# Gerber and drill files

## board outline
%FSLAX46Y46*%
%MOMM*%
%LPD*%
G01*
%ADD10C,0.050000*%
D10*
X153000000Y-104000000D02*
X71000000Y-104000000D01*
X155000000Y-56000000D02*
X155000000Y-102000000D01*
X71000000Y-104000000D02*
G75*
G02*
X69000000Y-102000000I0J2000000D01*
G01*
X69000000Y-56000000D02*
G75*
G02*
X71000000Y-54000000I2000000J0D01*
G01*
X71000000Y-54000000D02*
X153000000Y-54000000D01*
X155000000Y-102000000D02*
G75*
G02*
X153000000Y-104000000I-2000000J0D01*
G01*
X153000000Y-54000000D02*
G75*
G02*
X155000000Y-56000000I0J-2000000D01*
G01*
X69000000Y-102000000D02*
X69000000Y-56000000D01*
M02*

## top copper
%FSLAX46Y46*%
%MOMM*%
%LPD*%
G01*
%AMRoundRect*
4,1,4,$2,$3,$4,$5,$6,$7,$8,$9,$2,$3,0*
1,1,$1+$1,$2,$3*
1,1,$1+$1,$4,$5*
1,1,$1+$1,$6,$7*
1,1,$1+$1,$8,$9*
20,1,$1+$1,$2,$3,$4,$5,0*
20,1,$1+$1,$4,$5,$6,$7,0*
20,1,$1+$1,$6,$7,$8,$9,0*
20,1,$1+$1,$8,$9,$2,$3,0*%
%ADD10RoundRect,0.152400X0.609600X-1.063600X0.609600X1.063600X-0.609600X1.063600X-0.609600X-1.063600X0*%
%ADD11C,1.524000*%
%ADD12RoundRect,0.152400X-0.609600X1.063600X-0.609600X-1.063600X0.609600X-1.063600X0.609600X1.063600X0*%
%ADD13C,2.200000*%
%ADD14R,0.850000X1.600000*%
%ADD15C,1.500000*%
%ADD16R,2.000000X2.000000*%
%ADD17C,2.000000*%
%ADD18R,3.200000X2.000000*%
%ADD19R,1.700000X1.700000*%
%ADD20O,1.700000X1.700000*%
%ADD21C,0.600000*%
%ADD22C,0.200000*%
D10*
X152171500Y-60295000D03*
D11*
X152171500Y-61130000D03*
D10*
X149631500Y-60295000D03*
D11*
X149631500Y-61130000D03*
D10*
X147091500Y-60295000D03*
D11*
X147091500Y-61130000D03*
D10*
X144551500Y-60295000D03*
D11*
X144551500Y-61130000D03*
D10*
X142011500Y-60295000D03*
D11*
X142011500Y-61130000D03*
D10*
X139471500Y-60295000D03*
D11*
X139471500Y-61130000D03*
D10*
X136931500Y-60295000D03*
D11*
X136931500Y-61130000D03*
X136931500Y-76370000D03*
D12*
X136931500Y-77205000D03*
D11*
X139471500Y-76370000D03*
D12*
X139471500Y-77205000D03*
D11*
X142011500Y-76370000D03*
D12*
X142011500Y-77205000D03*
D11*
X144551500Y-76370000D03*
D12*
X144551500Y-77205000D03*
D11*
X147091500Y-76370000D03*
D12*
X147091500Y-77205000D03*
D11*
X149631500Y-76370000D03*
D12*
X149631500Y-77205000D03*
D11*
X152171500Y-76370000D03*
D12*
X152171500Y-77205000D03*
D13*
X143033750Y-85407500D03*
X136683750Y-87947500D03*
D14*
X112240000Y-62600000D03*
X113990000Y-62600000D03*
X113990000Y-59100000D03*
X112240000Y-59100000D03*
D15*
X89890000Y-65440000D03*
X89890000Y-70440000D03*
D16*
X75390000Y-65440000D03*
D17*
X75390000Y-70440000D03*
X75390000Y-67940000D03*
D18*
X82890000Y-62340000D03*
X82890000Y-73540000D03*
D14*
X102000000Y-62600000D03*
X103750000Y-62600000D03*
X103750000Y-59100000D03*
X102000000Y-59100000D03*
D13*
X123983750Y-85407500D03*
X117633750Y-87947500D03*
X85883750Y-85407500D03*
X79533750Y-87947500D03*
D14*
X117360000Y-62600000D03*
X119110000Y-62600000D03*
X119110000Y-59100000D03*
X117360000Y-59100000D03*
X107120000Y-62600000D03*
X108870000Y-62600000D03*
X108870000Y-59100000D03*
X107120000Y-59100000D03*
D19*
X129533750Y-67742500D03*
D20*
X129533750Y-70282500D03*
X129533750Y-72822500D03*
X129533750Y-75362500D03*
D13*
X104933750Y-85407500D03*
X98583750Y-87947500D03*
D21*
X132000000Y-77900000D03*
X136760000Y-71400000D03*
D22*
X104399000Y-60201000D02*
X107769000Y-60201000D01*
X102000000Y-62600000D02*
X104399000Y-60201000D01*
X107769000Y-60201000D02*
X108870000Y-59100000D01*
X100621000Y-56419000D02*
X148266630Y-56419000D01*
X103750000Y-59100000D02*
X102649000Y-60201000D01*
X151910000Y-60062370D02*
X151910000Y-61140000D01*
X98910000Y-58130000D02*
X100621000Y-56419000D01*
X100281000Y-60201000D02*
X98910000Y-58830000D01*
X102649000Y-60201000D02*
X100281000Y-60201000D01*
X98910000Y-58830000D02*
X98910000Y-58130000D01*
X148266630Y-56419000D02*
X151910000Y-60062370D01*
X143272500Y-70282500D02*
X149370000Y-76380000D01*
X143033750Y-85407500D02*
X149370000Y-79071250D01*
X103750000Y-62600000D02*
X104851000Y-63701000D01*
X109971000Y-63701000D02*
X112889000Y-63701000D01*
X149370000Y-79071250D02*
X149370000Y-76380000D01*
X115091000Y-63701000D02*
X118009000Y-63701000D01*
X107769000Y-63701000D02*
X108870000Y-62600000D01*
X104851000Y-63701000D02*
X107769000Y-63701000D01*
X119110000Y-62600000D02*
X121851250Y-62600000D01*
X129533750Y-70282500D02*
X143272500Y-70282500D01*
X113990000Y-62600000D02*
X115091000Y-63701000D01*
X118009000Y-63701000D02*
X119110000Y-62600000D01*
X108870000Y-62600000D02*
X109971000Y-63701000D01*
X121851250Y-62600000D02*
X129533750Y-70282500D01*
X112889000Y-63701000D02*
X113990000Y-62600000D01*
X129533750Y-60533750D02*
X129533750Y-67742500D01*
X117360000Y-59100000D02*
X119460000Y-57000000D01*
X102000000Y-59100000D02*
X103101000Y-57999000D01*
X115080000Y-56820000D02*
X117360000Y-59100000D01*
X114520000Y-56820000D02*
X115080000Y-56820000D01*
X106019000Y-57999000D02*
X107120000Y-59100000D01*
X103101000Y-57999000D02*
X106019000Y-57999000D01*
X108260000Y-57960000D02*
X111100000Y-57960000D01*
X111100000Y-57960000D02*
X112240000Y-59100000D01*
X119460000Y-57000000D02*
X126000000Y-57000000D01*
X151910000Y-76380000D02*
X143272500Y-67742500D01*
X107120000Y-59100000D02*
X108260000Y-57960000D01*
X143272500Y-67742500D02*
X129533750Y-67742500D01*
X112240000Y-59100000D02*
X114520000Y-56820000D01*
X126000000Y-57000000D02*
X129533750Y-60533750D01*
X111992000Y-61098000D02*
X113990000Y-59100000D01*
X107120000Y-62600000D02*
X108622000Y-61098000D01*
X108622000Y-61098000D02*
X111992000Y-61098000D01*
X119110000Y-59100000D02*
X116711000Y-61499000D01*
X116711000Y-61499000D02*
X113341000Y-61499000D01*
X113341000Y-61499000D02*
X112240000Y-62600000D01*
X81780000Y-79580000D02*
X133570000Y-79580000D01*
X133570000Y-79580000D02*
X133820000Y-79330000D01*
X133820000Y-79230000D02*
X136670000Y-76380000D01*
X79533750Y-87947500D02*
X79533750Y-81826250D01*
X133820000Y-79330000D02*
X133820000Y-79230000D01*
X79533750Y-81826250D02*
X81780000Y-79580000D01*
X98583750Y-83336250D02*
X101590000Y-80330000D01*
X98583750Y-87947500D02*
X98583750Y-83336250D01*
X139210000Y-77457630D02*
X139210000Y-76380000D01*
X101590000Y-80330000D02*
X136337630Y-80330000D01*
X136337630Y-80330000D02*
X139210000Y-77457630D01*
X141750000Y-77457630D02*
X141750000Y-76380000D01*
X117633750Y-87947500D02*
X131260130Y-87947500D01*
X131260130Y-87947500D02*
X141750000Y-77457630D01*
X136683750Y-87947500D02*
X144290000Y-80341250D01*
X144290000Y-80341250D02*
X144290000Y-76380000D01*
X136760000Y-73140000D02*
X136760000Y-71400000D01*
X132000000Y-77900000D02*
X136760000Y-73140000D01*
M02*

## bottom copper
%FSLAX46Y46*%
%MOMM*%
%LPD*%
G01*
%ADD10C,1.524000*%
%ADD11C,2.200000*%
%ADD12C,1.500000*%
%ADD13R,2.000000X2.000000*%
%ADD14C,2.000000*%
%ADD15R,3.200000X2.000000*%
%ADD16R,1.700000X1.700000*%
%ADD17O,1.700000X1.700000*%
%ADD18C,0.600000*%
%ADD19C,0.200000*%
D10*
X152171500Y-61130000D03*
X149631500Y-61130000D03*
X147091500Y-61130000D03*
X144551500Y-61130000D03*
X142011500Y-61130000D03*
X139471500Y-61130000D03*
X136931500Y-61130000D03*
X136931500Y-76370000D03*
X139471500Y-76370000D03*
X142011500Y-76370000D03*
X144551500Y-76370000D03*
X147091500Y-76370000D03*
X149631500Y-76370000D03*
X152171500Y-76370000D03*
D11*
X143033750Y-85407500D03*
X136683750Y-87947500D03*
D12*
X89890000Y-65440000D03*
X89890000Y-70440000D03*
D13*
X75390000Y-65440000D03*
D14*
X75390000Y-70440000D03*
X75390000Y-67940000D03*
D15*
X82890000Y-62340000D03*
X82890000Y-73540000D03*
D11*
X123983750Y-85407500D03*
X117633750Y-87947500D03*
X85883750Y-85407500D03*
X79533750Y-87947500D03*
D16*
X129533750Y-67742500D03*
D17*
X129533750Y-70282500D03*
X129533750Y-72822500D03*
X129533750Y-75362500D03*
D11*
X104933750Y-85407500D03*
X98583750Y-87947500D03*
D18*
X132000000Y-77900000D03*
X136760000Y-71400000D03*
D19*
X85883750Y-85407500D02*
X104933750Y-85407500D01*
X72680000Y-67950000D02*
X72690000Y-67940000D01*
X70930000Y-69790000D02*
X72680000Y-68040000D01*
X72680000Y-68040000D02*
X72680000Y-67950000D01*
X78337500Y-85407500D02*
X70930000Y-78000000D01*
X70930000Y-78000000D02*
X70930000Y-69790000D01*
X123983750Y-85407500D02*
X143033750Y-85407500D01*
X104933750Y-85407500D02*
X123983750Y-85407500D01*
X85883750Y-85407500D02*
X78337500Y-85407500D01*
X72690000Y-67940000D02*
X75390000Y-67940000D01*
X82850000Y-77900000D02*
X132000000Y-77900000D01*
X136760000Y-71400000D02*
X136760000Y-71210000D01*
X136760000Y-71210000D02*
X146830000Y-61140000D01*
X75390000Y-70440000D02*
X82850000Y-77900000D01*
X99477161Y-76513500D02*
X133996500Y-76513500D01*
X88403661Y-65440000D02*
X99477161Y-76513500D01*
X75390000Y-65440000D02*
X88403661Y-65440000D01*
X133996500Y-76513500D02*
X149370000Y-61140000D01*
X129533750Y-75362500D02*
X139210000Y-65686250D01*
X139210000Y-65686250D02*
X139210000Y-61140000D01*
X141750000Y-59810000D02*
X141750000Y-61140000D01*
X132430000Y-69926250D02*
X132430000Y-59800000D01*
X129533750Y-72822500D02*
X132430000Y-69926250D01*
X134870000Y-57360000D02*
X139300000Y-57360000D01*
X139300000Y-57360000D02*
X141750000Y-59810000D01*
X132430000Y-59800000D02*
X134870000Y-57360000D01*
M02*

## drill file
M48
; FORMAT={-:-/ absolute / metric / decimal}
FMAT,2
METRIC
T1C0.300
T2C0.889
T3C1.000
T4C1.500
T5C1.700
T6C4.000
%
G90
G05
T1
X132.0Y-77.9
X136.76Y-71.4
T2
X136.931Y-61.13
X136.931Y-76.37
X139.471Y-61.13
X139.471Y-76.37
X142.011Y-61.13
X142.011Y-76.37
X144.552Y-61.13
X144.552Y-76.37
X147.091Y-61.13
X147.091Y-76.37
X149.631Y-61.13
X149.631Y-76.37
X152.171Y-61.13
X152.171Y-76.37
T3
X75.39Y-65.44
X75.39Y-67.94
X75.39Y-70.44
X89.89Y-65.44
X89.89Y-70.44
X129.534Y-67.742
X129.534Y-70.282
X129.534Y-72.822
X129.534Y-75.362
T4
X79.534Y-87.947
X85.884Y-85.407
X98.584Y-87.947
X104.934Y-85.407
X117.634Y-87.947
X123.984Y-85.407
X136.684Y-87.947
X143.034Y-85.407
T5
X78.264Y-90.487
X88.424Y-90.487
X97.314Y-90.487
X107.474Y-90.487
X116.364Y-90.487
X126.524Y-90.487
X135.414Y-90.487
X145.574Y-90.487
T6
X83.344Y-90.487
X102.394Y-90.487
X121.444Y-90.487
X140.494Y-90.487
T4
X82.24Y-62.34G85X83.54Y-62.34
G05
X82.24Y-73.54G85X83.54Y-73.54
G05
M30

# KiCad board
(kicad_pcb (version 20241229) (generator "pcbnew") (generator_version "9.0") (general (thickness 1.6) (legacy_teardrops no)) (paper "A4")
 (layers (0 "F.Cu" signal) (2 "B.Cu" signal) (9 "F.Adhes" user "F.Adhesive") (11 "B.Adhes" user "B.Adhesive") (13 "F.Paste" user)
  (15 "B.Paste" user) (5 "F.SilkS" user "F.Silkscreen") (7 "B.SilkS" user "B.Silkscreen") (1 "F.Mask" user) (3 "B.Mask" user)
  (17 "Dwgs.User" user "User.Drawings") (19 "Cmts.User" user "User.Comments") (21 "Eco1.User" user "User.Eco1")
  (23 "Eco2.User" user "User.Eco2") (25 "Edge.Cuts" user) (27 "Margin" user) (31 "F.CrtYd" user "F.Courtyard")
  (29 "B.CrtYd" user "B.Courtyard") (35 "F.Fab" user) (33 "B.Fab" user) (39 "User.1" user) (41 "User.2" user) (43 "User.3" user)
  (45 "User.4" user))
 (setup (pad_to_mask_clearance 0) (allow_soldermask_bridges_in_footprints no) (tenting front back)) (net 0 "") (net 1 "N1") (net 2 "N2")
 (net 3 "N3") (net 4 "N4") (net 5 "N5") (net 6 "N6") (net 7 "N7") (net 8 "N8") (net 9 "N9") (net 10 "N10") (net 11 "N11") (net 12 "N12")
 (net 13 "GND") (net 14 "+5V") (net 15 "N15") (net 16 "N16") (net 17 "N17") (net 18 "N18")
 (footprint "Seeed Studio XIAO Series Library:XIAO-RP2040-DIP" (layer "F.Cu") (at 144.5515 68.75 -90)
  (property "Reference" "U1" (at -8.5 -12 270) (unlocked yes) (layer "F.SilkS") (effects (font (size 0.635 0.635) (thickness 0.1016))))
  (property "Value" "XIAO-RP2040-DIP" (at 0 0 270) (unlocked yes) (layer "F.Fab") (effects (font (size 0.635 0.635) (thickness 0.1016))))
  (pad "1" smd roundrect (at -8.455 -7.62 90) (size 2.432 1.524) (layers "F.Cu" "F.Mask") (roundrect_rratio 0.1) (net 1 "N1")
   (thermal_bridge_angle 45))
  (pad "1" thru_hole circle (at -7.62 -7.62 90) (size 1.524 1.524) (drill 0.889) (layers "*.Cu" "*.Mask") (remove_unused_layers no)
   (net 1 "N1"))
  (pad "2" smd roundrect (at -8.455 -5.08 90) (size 2.432 1.524) (layers "F.Cu" "F.Mask") (roundrect_rratio 0.1) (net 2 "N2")
   (thermal_bridge_angle 45))
  (pad "2" thru_hole circle (at -7.62 -5.08 90) (size 1.524 1.524) (drill 0.889) (layers "*.Cu" "*.Mask") (remove_unused_layers no)
   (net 2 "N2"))
  (pad "3" smd roundrect (at -8.455 -2.54 90) (size 2.432 1.524) (layers "F.Cu" "F.Mask") (roundrect_rratio 0.1) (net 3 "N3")
   (thermal_bridge_angle 45))
  (pad "3" thru_hole circle (at -7.62 -2.54 90) (size 1.524 1.524) (drill 0.889) (layers "*.Cu" "*.Mask") (remove_unused_layers no)
   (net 3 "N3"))
  (pad "4" smd roundrect (at -8.455 0 90) (size 2.432 1.524) (layers "F.Cu" "F.Mask") (roundrect_rratio 0.1) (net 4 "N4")
   (thermal_bridge_angle 45))
  (pad "4" thru_hole circle (at -7.62 0 90) (size 1.524 1.524) (drill 0.889) (layers "*.Cu" "*.Mask") (remove_unused_layers no) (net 4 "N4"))
  (pad "5" smd roundrect (at -8.455 2.54 90) (size 2.432 1.524) (layers "F.Cu" "F.Mask") (roundrect_rratio 0.1) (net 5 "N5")
   (thermal_bridge_angle 45))
  (pad "5" thru_hole circle (at -7.62 2.54 90) (size 1.524 1.524) (drill 0.889) (layers "*.Cu" "*.Mask") (remove_unused_layers no)
   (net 5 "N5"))
  (pad "6" smd roundrect (at -8.455 5.08 90) (size 2.432 1.524) (layers "F.Cu" "F.Mask") (roundrect_rratio 0.1) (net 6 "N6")
   (thermal_bridge_angle 45))
  (pad "6" thru_hole circle (at -7.62 5.08 90) (size 1.524 1.524) (drill 0.889) (layers "*.Cu" "*.Mask") (remove_unused_layers no)
   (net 6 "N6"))
  (pad "7" smd roundrect (at -8.455 7.62 90) (size 2.432 1.524) (layers "F.Cu" "F.Mask") (roundrect_rratio 0.1) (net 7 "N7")
   (thermal_bridge_angle 45))
  (pad "7" thru_hole circle (at -7.62 7.62 90) (size 1.524 1.524) (drill 0.889) (layers "*.Cu" "*.Mask") (remove_unused_layers no)
   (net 7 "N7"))
  (pad "8" thru_hole circle (at 7.62 7.62 270) (size 1.524 1.524) (drill 0.889) (layers "*.Cu" "*.Mask") (remove_unused_layers no)
   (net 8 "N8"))
  (pad "8" smd roundrect (at 8.455 7.62 270) (size 2.432 1.524) (layers "F.Cu" "F.Mask") (roundrect_rratio 0.1) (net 8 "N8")
   (thermal_bridge_angle 45))
  (pad "9" thru_hole circle (at 7.62 5.08 270) (size 1.524 1.524) (drill 0.889) (layers "*.Cu" "*.Mask") (remove_unused_layers no)
   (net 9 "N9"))
  (pad "9" smd roundrect (at 8.455 5.08 270) (size 2.432 1.524) (layers "F.Cu" "F.Mask") (roundrect_rratio 0.1) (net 9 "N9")
   (thermal_bridge_angle 45))
  (pad "10" thru_hole circle (at 7.62 2.54 270) (size 1.524 1.524) (drill 0.889) (layers "*.Cu" "*.Mask") (remove_unused_layers no)
   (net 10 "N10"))
  (pad "10" smd roundrect (at 8.455 2.54 270) (size 2.432 1.524) (layers "F.Cu" "F.Mask") (roundrect_rratio 0.1) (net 10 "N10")
   (thermal_bridge_angle 45))
  (pad "11" thru_hole circle (at 7.62 0 270) (size 1.524 1.524) (drill 0.889) (layers "*.Cu" "*.Mask") (remove_unused_layers no)
   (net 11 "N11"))
  (pad "11" smd roundrect (at 8.455 0 270) (size 2.432 1.524) (layers "F.Cu" "F.Mask") (roundrect_rratio 0.1) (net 11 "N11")
   (thermal_bridge_angle 45))
  (pad "12" thru_hole circle (at 7.62 -2.54 270) (size 1.524 1.524) (drill 0.889) (layers "*.Cu" "*.Mask") (remove_unused_layers no)
   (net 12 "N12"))
  (pad "12" smd roundrect (at 8.455 -2.54 270) (size 2.432 1.524) (layers "F.Cu" "F.Mask") (roundrect_rratio 0.1) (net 12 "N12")
   (thermal_bridge_angle 45))
  (pad "13" thru_hole circle (at 7.62 -5.08 270) (size 1.524 1.524) (drill 0.889) (layers "*.Cu" "*.Mask") (remove_unused_layers no)
   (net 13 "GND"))
  (pad "13" smd roundrect (at 8.455 -5.08 270) (size 2.432 1.524) (layers "F.Cu" "F.Mask") (roundrect_rratio 0.1) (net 13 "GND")
   (thermal_bridge_angle 45))
  (pad "14" thru_hole circle (at 7.62 -7.62 270) (size 1.524 1.524) (drill 0.889) (layers "*.Cu" "*.Mask") (remove_unused_layers no)
   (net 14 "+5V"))
  (pad "14" smd roundrect (at 8.455 -7.62 270) (size 2.432 1.524) (layers "F.Cu" "F.Mask") (roundrect_rratio 0.1) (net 14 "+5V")
   (thermal_bridge_angle 45)))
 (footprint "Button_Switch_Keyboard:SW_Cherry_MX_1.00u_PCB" (layer "F.Cu") (at 143.03375 85.4075)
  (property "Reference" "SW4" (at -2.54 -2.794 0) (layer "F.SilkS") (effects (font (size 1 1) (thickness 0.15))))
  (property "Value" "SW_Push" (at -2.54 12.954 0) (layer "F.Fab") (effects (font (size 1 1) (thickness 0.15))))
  (pad "" np_thru_hole circle (at -7.62 5.08) (size 1.7 1.7) (drill 1.7) (layers "*.Cu" "*.Mask"))
  (pad "" np_thru_hole circle (at -2.54 5.08) (size 4 4) (drill 4) (layers "*.Cu" "*.Mask"))
  (pad "" np_thru_hole circle (at 2.54 5.08) (size 1.7 1.7) (drill 1.7) (layers "*.Cu" "*.Mask"))
  (pad "1" thru_hole circle (at 0 0) (size 2.2 2.2) (drill 1.5) (layers "*.Cu" "*.Mask") (remove_unused_layers no) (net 13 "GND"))
  (pad "2" thru_hole circle (at -6.35 2.54) (size 2.2 2.2) (drill 1.5) (layers "*.Cu" "*.Mask") (remove_unused_layers no) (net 11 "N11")))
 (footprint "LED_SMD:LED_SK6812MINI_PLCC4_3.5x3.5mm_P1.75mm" (layer "F.Cu") (at 113.115 60.85 90)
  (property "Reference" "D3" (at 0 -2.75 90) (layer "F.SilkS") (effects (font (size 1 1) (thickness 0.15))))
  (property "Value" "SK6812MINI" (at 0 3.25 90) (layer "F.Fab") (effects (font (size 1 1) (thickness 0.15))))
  (pad "1" smd rect (at -1.75 -0.875 90) (size 1.6 0.85) (layers "F.Cu" "F.Mask" "F.Paste") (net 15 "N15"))
  (pad "2" smd rect (at -1.75 0.875 90) (size 1.6 0.85) (layers "F.Cu" "F.Mask" "F.Paste") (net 13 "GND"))
  (pad "3" smd rect (at 1.75 0.875 90) (size 1.6 0.85) (layers "F.Cu" "F.Mask" "F.Paste") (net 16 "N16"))
  (pad "4" smd rect (at 1.75 -0.875 90) (size 1.6 0.85) (layers "F.Cu" "F.Mask" "F.Paste") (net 14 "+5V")))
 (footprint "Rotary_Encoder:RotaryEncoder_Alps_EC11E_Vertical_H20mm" (layer "F.Cu") (at 75.39 65.44)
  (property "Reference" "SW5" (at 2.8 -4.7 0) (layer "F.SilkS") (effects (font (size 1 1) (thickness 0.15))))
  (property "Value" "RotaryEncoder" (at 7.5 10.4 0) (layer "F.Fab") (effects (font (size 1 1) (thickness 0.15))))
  (pad "" thru_hole circle (at 14.5 0) (size 1.5 1.5) (drill 1) (layers "*.Cu" "*.Mask") (remove_unused_layers no))
  (pad "" thru_hole circle (at 14.5 5) (size 1.5 1.5) (drill 1) (layers "*.Cu" "*.Mask") (remove_unused_layers no))
  (pad "A" thru_hole rect (at 0 0) (size 2 2) (drill 1) (layers "*.Cu" "*.Mask") (remove_unused_layers no) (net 2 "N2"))
  (pad "B" thru_hole circle (at 0 5) (size 2 2) (drill 1) (layers "*.Cu" "*.Mask") (remove_unused_layers no) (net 3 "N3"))
  (pad "C" thru_hole circle (at 0 2.5) (size 2 2) (drill 1) (layers "*.Cu" "*.Mask") (remove_unused_layers no) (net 13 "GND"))
  (pad "MP" thru_hole rect (at 7.5 -3.1) (size 3.2 2) (drill oval 2.8 1.5) (layers "*.Cu" "*.Mask") (remove_unused_layers no))
  (pad "MP" thru_hole rect (at 7.5 8.1) (size 3.2 2) (drill oval 2.8 1.5) (layers "*.Cu" "*.Mask") (remove_unused_layers no)))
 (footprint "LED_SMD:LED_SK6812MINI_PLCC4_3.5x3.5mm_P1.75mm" (layer "F.Cu") (at 102.875 60.85 90)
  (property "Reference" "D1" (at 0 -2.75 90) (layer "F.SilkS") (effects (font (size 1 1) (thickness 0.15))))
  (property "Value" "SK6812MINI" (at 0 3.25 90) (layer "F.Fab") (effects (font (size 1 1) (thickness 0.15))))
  (pad "1" smd rect (at -1.75 -0.875 90) (size 1.6 0.85) (layers "F.Cu" "F.Mask" "F.Paste") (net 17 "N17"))
  (pad "2" smd rect (at -1.75 0.875 90) (size 1.6 0.85) (layers "F.Cu" "F.Mask" "F.Paste") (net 13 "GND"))
  (pad "3" smd rect (at 1.75 0.875 90) (size 1.6 0.85) (layers "F.Cu" "F.Mask" "F.Paste") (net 1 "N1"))
  (pad "4" smd rect (at 1.75 -0.875 90) (size 1.6 0.85) (layers "F.Cu" "F.Mask" "F.Paste") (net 14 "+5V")))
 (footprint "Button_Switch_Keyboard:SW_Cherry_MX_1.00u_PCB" (layer "F.Cu") (at 123.98375 85.4075)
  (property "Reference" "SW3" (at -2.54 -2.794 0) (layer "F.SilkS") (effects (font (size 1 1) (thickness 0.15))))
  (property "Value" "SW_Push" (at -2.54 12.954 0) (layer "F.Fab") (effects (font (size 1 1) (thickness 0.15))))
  (pad "" np_thru_hole circle (at -7.62 5.08) (size 1.7 1.7) (drill 1.7) (layers "*.Cu" "*.Mask"))
  (pad "" np_thru_hole circle (at -2.54 5.08) (size 4 4) (drill 4) (layers "*.Cu" "*.Mask"))
  (pad "" np_thru_hole circle (at 2.54 5.08) (size 1.7 1.7) (drill 1.7) (layers "*.Cu" "*.Mask"))
  (pad "1" thru_hole circle (at 0 0) (size 2.2 2.2) (drill 1.5) (layers "*.Cu" "*.Mask") (remove_unused_layers no) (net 13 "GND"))
  (pad "2" thru_hole circle (at -6.35 2.54) (size 2.2 2.2) (drill 1.5) (layers "*.Cu" "*.Mask") (remove_unused_layers no) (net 10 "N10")))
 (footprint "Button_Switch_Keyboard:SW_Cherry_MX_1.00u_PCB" (layer "F.Cu") (at 85.88375 85.4075)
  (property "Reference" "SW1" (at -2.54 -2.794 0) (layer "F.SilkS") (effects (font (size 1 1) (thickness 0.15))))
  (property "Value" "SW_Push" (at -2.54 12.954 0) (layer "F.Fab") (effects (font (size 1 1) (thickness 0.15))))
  (pad "" np_thru_hole circle (at -7.62 5.08) (size 1.7 1.7) (drill 1.7) (layers "*.Cu" "*.Mask"))
  (pad "" np_thru_hole circle (at -2.54 5.08) (size 4 4) (drill 4) (layers "*.Cu" "*.Mask"))
  (pad "" np_thru_hole circle (at 2.54 5.08) (size 1.7 1.7) (drill 1.7) (layers "*.Cu" "*.Mask"))
  (pad "1" thru_hole circle (at 0 0) (size 2.2 2.2) (drill 1.5) (layers "*.Cu" "*.Mask") (remove_unused_layers no) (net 13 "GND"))
  (pad "2" thru_hole circle (at -6.35 2.54) (size 2.2 2.2) (drill 1.5) (layers "*.Cu" "*.Mask") (remove_unused_layers no) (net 8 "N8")))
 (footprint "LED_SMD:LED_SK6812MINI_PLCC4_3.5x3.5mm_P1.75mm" (layer "F.Cu") (at 118.235 60.85 90)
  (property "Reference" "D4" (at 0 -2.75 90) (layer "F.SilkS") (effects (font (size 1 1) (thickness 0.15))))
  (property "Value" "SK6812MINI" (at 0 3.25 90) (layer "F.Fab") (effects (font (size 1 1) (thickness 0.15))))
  (pad "1" smd rect (at -1.75 -0.875 90) (size 1.6 0.85) (layers "F.Cu" "F.Mask" "F.Paste") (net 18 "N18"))
  (pad "2" smd rect (at -1.75 0.875 90) (size 1.6 0.85) (layers "F.Cu" "F.Mask" "F.Paste") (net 13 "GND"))
  (pad "3" smd rect (at 1.75 0.875 90) (size 1.6 0.85) (layers "F.Cu" "F.Mask" "F.Paste") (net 15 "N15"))
  (pad "4" smd rect (at 1.75 -0.875 90) (size 1.6 0.85) (layers "F.Cu" "F.Mask" "F.Paste") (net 14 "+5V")))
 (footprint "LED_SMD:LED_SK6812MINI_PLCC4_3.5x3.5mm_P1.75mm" (layer "F.Cu") (at 107.995 60.85 90)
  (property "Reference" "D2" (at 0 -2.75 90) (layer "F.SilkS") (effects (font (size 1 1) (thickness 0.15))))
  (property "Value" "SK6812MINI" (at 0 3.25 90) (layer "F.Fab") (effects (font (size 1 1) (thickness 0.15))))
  (pad "1" smd rect (at -1.75 -0.875 90) (size 1.6 0.85) (layers "F.Cu" "F.Mask" "F.Paste") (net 16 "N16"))
  (pad "2" smd rect (at -1.75 0.875 90) (size 1.6 0.85) (layers "F.Cu" "F.Mask" "F.Paste") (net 13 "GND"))
  (pad "3" smd rect (at 1.75 0.875 90) (size 1.6 0.85) (layers "F.Cu" "F.Mask" "F.Paste") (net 17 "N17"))
  (pad "4" smd rect (at 1.75 -0.875 90) (size 1.6 0.85) (layers "F.Cu" "F.Mask" "F.Paste") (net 14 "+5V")))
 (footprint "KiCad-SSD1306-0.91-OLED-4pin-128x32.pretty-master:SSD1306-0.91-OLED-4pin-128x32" (layer "F.Cu") (at 93.03375 65.5525)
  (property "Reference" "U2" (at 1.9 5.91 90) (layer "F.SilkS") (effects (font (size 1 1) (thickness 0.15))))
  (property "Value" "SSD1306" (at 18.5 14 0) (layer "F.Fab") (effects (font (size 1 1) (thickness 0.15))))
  (pad "1" thru_hole rect (at 36.5 2.19) (size 1.7 1.7) (drill 1) (layers "*.Cu" "*.Mask") (remove_unused_layers no) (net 14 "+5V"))
  (pad "2" thru_hole oval (at 36.5 4.73) (size 1.7 1.7) (drill 1) (layers "*.Cu" "*.Mask") (remove_unused_layers no) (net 13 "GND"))
  (pad "3" thru_hole oval (at 36.5 7.27) (size 1.7 1.7) (drill 1) (layers "*.Cu" "*.Mask") (remove_unused_layers no) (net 5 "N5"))
  (pad "4" thru_hole oval (at 36.5 9.81) (size 1.7 1.7) (drill 1) (layers "*.Cu" "*.Mask") (remove_unused_layers no) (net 6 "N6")))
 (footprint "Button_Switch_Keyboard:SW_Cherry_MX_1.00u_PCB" (layer "F.Cu") (at 104.93375 85.4075)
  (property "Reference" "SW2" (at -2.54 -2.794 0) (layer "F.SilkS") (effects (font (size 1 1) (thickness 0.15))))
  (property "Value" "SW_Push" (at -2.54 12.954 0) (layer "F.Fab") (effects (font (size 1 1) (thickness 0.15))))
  (pad "" np_thru_hole circle (at -7.62 5.08) (size 1.7 1.7) (drill 1.7) (layers "*.Cu" "*.Mask"))
  (pad "" np_thru_hole circle (at -2.54 5.08) (size 4 4) (drill 4) (layers "*.Cu" "*.Mask"))
  (pad "" np_thru_hole circle (at 2.54 5.08) (size 1.7 1.7) (drill 1.7) (layers "*.Cu" "*.Mask"))
  (pad "1" thru_hole circle (at 0 0) (size 2.2 2.2) (drill 1.5) (layers "*.Cu" "*.Mask") (remove_unused_layers no) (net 13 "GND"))
  (pad "2" thru_hole circle (at -6.35 2.54) (size 2.2 2.2) (drill 1.5) (layers "*.Cu" "*.Mask") (remove_unused_layers no) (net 9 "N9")))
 (gr_line (start 153 104) (end 71 104) (stroke (width 0.05) (type default)) (layer "Edge.Cuts"))
 (gr_line (start 155 56) (end 155 102) (stroke (width 0.05) (type default)) (layer "Edge.Cuts"))
 (gr_arc (start 71 104) (mid 69.585786 103.414214) (end 69 102) (stroke (width 0.05) (type default)) (layer "Edge.Cuts"))
 (gr_arc (start 69 56) (mid 69.585786 54.585786) (end 71 54) (stroke (width 0.05) (type default)) (layer "Edge.Cuts"))
 (gr_line (start 71 54) (end 153 54) (stroke (width 0.05) (type default)) (layer "Edge.Cuts"))
 (gr_arc (start 155 102) (mid 154.414214 103.414214) (end 153 104) (stroke (width 0.05) (type default)) (layer "Edge.Cuts"))
 (gr_arc (start 153 54) (mid 154.414214 54.585786) (end 155 56) (stroke (width 0.05) (type default)) (layer "Edge.Cuts"))
 (gr_line (start 69 102) (end 69 56) (stroke (width 0.05) (type default)) (layer "Edge.Cuts"))
 (segment (start 104.399 60.201) (end 107.769 60.201) (width 0.2) (layer "F.Cu") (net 17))
 (segment (start 102 62.6) (end 104.399 60.201) (width 0.2) (layer "F.Cu") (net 17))
 (segment (start 107.769 60.201) (end 108.87 59.1) (width 0.2) (layer "F.Cu") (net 17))
 (segment (start 100.621 56.419) (end 148.26663 56.419) (width 0.2) (layer "F.Cu") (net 1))
 (segment (start 103.75 59.1) (end 102.649 60.201) (width 0.2) (layer "F.Cu") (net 1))
 (segment (start 151.91 60.06237) (end 151.91 61.14) (width 0.2) (layer "F.Cu") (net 1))
 (segment (start 98.91 58.13) (end 100.621 56.419) (width 0.2) (layer "F.Cu") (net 1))
 (segment (start 100.281 60.201) (end 98.91 58.83) (width 0.2) (layer "F.Cu") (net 1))
 (segment (start 102.649 60.201) (end 100.281 60.201) (width 0.2) (layer "F.Cu") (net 1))
 (segment (start 98.91 58.83) (end 98.91 58.13) (width 0.2) (layer "F.Cu") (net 1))
 (segment (start 148.26663 56.419) (end 151.91 60.06237) (width 0.2) (layer "F.Cu") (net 1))
 (segment (start 143.2725 70.2825) (end 149.37 76.38) (width 0.2) (layer "F.Cu") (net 13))
 (segment (start 143.03375 85.4075) (end 149.37 79.07125) (width 0.2) (layer "F.Cu") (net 13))
 (segment (start 103.75 62.6) (end 104.851 63.701) (width 0.2) (layer "F.Cu") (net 13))
 (segment (start 109.971 63.701) (end 112.889 63.701) (width 0.2) (layer "F.Cu") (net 13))
 (segment (start 149.37 79.07125) (end 149.37 76.38) (width 0.2) (layer "F.Cu") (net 13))
 (segment (start 115.091 63.701) (end 118.009 63.701) (width 0.2) (layer "F.Cu") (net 13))
 (segment (start 107.769 63.701) (end 108.87 62.6) (width 0.2) (layer "F.Cu") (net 13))
 (segment (start 104.851 63.701) (end 107.769 63.701) (width 0.2) (layer "F.Cu") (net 13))
 (segment (start 119.11 62.6) (end 121.85125 62.6) (width 0.2) (layer "F.Cu") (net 13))
 (segment (start 129.53375 70.2825) (end 143.2725 70.2825) (width 0.2) (layer "F.Cu") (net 13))
 (segment (start 113.99 62.6) (end 115.091 63.701) (width 0.2) (layer "F.Cu") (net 13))
 (segment (start 118.009 63.701) (end 119.11 62.6) (width 0.2) (layer "F.Cu") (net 13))
 (segment (start 108.87 62.6) (end 109.971 63.701) (width 0.2) (layer "F.Cu") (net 13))
 (segment (start 121.85125 62.6) (end 129.53375 70.2825) (width 0.2) (layer "F.Cu") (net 13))
 (segment (start 112.889 63.701) (end 113.99 62.6) (width 0.2) (layer "F.Cu") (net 13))
 (segment (start 85.88375 85.4075) (end 104.93375 85.4075) (width 0.2) (layer "B.Cu") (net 13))
 (segment (start 72.68 67.95) (end 72.69 67.94) (width 0.2) (layer "B.Cu") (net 13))
 (segment (start 70.93 69.79) (end 72.68 68.04) (width 0.2) (layer "B.Cu") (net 13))
 (segment (start 72.68 68.04) (end 72.68 67.95) (width 0.2) (layer "B.Cu") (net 13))
 (segment (start 78.3375 85.4075) (end 70.93 78) (width 0.2) (layer "B.Cu") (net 13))
 (segment (start 70.93 78) (end 70.93 69.79) (width 0.2) (layer "B.Cu") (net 13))
 (segment (start 123.98375 85.4075) (end 143.03375 85.4075) (width 0.2) (layer "B.Cu") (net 13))
 (segment (start 104.93375 85.4075) (end 123.98375 85.4075) (width 0.2) (layer "B.Cu") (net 13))
 (segment (start 85.88375 85.4075) (end 78.3375 85.4075) (width 0.2) (layer "B.Cu") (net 13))
 (segment (start 72.69 67.94) (end 75.39 67.94) (width 0.2) (layer "B.Cu") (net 13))
 (segment (start 129.53375 60.53375) (end 129.53375 67.7425) (width 0.2) (layer "F.Cu") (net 14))
 (segment (start 117.36 59.1) (end 119.46 57) (width 0.2) (layer "F.Cu") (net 14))
 (segment (start 102 59.1) (end 103.101 57.999) (width 0.2) (layer "F.Cu") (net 14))
 (segment (start 115.08 56.82) (end 117.36 59.1) (width 0.2) (layer "F.Cu") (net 14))
 (segment (start 114.52 56.82) (end 115.08 56.82) (width 0.2) (layer "F.Cu") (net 14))
 (segment (start 106.019 57.999) (end 107.12 59.1) (width 0.2) (layer "F.Cu") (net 14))
 (segment (start 103.101 57.999) (end 106.019 57.999) (width 0.2) (layer "F.Cu") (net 14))
 (segment (start 108.26 57.96) (end 111.1 57.96) (width 0.2) (layer "F.Cu") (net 14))
 (segment (start 111.1 57.96) (end 112.24 59.1) (width 0.2) (layer "F.Cu") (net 14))
 (segment (start 119.46 57) (end 126 57) (width 0.2) (layer "F.Cu") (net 14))
 (segment (start 151.91 76.38) (end 143.2725 67.7425) (width 0.2) (layer "F.Cu") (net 14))
 (segment (start 107.12 59.1) (end 108.26 57.96) (width 0.2) (layer "F.Cu") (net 14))
 (segment (start 143.2725 67.7425) (end 129.53375 67.7425) (width 0.2) (layer "F.Cu") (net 14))
 (segment (start 112.24 59.1) (end 114.52 56.82) (width 0.2) (layer "F.Cu") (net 14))
 (segment (start 126 57) (end 129.53375 60.53375) (width 0.2) (layer "F.Cu") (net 14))
 (segment (start 111.992 61.098) (end 113.99 59.1) (width 0.2) (layer "F.Cu") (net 16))
 (segment (start 107.12 62.6) (end 108.622 61.098) (width 0.2) (layer "F.Cu") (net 16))
 (segment (start 108.622 61.098) (end 111.992 61.098) (width 0.2) (layer "F.Cu") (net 16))
 (segment (start 119.11 59.1) (end 116.711 61.499) (width 0.2) (layer "F.Cu") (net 15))
 (segment (start 116.711 61.499) (end 113.341 61.499) (width 0.2) (layer "F.Cu") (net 15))
 (segment (start 113.341 61.499) (end 112.24 62.6) (width 0.2) (layer "F.Cu") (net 15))
 (segment (start 81.78 79.58) (end 133.57 79.58) (width 0.2) (layer "F.Cu") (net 8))
 (segment (start 133.57 79.58) (end 133.82 79.33) (width 0.2) (layer "F.Cu") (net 8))
 (segment (start 133.82 79.23) (end 136.67 76.38) (width 0.2) (layer "F.Cu") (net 8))
 (segment (start 79.53375 87.9475) (end 79.53375 81.82625) (width 0.2) (layer "F.Cu") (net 8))
 (segment (start 133.82 79.33) (end 133.82 79.23) (width 0.2) (layer "F.Cu") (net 8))
 (segment (start 79.53375 81.82625) (end 81.78 79.58) (width 0.2) (layer "F.Cu") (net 8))
 (segment (start 98.58375 83.33625) (end 101.59 80.33) (width 0.2) (layer "F.Cu") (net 9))
 (segment (start 98.58375 87.9475) (end 98.58375 83.33625) (width 0.2) (layer "F.Cu") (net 9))
 (segment (start 139.21 77.45763) (end 139.21 76.38) (width 0.2) (layer "F.Cu") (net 9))
 (segment (start 101.59 80.33) (end 136.33763 80.33) (width 0.2) (layer "F.Cu") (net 9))
 (segment (start 136.33763 80.33) (end 139.21 77.45763) (width 0.2) (layer "F.Cu") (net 9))
 (segment (start 141.75 77.45763) (end 141.75 76.38) (width 0.2) (layer "F.Cu") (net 10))
 (segment (start 117.63375 87.9475) (end 131.26013 87.9475) (width 0.2) (layer "F.Cu") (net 10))
 (segment (start 131.26013 87.9475) (end 141.75 77.45763) (width 0.2) (layer "F.Cu") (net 10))
 (segment (start 136.68375 87.9475) (end 144.29 80.34125) (width 0.2) (layer "F.Cu") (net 11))
 (segment (start 144.29 80.34125) (end 144.29 76.38) (width 0.2) (layer "F.Cu") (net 11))
 (segment (start 136.76 73.14) (end 136.76 71.4) (width 0.2) (layer "F.Cu") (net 3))
 (segment (start 132 77.9) (end 136.76 73.14) (width 0.2) (layer "F.Cu") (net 3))
 (via (at 132 77.9) (size 0.6) (drill 0.3) (layers "F.Cu" "B.Cu") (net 3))
 (via (at 136.76 71.4) (size 0.6) (drill 0.3) (layers "F.Cu" "B.Cu") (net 3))
 (segment (start 82.85 77.9) (end 132 77.9) (width 0.2) (layer "B.Cu") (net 3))
 (segment (start 136.76 71.4) (end 136.76 71.21) (width 0.2) (layer "B.Cu") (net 3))
 (segment (start 136.76 71.21) (end 146.83 61.14) (width 0.2) (layer "B.Cu") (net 3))
 (segment (start 75.39 70.44) (end 82.85 77.9) (width 0.2) (layer "B.Cu") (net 3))
 (segment (start 99.477161 76.5135) (end 133.9965 76.5135) (width 0.2) (layer "B.Cu") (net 2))
 (segment (start 88.403661 65.44) (end 99.477161 76.5135) (width 0.2) (layer "B.Cu") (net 2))
 (segment (start 75.39 65.44) (end 88.403661 65.44) (width 0.2) (layer "B.Cu") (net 2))
 (segment (start 133.9965 76.5135) (end 149.37 61.14) (width 0.2) (layer "B.Cu") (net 2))
 (segment (start 129.53375 75.3625) (end 139.21 65.68625) (width 0.2) (layer "B.Cu") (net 6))
 (segment (start 139.21 65.68625) (end 139.21 61.14) (width 0.2) (layer "B.Cu") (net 6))
 (segment (start 141.75 59.81) (end 141.75 61.14) (width 0.2) (layer "B.Cu") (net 5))
 (segment (start 132.43 69.92625) (end 132.43 59.8) (width 0.2) (layer "B.Cu") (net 5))
 (segment (start 129.53375 72.8225) (end 132.43 69.92625) (width 0.2) (layer "B.Cu") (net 5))
 (segment (start 134.87 57.36) (end 139.3 57.36) (width 0.2) (layer "B.Cu") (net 5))
 (segment (start 139.3 57.36) (end 141.75 59.81) (width 0.2) (layer "B.Cu") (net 5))
 (segment (start 132.43 59.8) (end 134.87 57.36) (width 0.2) (layer "B.Cu") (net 5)))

